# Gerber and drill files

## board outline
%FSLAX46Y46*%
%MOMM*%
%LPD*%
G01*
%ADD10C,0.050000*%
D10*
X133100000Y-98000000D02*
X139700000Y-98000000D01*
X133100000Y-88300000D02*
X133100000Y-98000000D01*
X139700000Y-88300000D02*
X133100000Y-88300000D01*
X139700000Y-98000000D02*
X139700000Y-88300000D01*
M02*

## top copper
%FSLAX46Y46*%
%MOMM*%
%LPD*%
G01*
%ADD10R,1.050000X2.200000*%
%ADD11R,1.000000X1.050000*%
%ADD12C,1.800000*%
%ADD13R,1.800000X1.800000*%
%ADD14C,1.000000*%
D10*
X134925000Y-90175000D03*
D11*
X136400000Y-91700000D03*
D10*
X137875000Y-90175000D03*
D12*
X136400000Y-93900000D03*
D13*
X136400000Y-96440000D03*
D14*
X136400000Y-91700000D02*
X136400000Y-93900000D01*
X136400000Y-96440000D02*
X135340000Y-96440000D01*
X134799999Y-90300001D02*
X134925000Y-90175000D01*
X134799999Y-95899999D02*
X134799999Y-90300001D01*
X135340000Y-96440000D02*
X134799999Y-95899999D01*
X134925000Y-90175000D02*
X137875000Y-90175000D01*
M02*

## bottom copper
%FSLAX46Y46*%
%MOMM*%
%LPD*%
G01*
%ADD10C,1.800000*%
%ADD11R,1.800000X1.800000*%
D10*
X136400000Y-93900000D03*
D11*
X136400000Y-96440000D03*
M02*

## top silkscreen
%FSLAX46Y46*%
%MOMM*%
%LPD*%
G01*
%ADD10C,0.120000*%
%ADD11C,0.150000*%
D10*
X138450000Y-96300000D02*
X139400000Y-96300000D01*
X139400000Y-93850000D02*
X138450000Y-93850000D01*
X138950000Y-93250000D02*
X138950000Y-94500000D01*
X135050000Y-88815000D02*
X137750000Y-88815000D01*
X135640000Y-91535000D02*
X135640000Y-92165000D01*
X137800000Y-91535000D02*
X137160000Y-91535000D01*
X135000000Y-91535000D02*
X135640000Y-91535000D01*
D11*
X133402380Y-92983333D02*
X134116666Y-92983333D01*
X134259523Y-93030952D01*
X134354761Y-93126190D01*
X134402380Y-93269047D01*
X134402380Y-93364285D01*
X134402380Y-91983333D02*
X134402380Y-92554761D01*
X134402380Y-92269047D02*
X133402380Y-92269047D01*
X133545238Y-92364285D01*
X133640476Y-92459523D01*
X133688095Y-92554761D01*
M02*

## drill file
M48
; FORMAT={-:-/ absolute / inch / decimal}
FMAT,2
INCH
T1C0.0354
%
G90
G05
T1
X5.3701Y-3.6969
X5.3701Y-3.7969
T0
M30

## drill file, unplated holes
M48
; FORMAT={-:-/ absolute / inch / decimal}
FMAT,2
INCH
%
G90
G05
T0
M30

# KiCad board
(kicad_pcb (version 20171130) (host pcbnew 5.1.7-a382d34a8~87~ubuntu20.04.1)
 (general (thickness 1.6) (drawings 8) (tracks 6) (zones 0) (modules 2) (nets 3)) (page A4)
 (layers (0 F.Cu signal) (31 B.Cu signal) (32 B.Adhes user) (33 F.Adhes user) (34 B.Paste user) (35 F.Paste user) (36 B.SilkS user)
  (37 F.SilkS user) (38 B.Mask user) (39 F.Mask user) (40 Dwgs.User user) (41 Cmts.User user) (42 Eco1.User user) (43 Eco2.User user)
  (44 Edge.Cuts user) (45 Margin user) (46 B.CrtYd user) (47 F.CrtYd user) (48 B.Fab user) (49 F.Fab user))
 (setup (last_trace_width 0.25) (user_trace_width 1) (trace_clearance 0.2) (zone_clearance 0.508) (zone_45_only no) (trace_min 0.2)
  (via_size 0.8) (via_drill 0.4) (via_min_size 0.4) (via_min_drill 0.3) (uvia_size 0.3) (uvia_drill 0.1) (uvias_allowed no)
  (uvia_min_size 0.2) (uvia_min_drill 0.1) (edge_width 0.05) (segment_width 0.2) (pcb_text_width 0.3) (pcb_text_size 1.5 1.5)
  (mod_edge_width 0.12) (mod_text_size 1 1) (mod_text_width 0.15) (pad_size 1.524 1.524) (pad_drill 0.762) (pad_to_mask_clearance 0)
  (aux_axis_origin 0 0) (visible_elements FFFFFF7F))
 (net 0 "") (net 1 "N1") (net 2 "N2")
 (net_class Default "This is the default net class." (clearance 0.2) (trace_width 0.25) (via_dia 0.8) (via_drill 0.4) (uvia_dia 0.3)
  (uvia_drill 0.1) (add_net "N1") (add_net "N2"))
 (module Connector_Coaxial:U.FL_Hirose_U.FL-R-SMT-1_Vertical (layer F.Cu) (at 136.4 90.65 90)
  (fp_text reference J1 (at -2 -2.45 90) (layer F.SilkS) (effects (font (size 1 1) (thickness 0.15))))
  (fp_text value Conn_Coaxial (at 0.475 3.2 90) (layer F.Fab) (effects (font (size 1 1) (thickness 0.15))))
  (fp_line (start 1.835 -1.35) (end 1.835 1.35) (layer F.SilkS) (width 0.12))
  (fp_line (start -0.885 -0.76) (end -1.515 -0.76) (layer F.SilkS) (width 0.12))
  (fp_line (start -0.885 1.4) (end -0.885 0.76) (layer F.SilkS) (width 0.12))
  (fp_line (start -0.885 -1.4) (end -0.885 -0.76) (layer F.SilkS) (width 0.12))
  (pad 2 smd rect (at 0.475 -1.475 90) (size 2.2 1.05) (layers F.Cu F.Paste F.Mask) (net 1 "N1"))
  (pad 1 smd rect (at -1.05 0 90) (size 1.05 1) (layers F.Cu F.Paste F.Mask) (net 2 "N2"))
  (pad 2 smd rect (at 0.475 1.475 90) (size 2.2 1.05) (layers F.Cu F.Paste F.Mask) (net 1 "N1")))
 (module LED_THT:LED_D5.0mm (layer B.Cu) (at 136.4 96.44 90)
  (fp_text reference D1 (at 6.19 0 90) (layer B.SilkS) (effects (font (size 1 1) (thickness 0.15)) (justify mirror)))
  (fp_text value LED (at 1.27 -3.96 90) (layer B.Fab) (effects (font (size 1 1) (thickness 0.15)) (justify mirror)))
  (pad 2 thru_hole circle (at 2.54 0 90) (size 1.8 1.8) (drill 0.9) (layers *.Cu *.Mask) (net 2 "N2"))
  (pad 1 thru_hole rect (at 0 0 90) (size 1.8 1.8) (drill 0.9) (layers *.Cu *.Mask) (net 1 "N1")))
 (gr_line (start 138.45 96.3) (end 139.4 96.3) (layer F.SilkS) (width 0.12))
 (gr_line (start 139.4 93.85) (end 138.45 93.85) (layer F.SilkS) (width 0.12))
 (gr_line (start 138.95 93.25) (end 138.95 94.5) (layer F.SilkS) (width 0.12))
 (gr_line (start 133.1 98) (end 139.7 98) (layer Edge.Cuts) (width 0.05))
 (gr_line (start 133.1 88.3) (end 133.1 98) (layer Edge.Cuts) (width 0.05))
 (gr_line (start 139.7 88.3) (end 133.1 88.3) (layer Edge.Cuts) (width 0.05))
 (gr_line (start 139.7 98) (end 139.7 88.3) (layer Edge.Cuts) (width 0.05))
 (segment (start 136.4 91.7) (end 136.4 93.9) (width 1) (layer F.Cu) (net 2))
 (segment (start 136.4 96.44) (end 135.34 96.44) (width 1) (layer F.Cu) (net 1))
 (segment (start 134.799999 90.300001) (end 134.925 90.175) (width 1) (layer F.Cu) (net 1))
 (segment (start 134.799999 95.899999) (end 134.799999 90.300001) (width 1) (layer F.Cu) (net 1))
 (segment (start 135.34 96.44) (end 134.799999 95.899999) (width 1) (layer F.Cu) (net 1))
 (segment (start 134.925 90.175) (end 137.875 90.175) (width 1) (layer F.Cu) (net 1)))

